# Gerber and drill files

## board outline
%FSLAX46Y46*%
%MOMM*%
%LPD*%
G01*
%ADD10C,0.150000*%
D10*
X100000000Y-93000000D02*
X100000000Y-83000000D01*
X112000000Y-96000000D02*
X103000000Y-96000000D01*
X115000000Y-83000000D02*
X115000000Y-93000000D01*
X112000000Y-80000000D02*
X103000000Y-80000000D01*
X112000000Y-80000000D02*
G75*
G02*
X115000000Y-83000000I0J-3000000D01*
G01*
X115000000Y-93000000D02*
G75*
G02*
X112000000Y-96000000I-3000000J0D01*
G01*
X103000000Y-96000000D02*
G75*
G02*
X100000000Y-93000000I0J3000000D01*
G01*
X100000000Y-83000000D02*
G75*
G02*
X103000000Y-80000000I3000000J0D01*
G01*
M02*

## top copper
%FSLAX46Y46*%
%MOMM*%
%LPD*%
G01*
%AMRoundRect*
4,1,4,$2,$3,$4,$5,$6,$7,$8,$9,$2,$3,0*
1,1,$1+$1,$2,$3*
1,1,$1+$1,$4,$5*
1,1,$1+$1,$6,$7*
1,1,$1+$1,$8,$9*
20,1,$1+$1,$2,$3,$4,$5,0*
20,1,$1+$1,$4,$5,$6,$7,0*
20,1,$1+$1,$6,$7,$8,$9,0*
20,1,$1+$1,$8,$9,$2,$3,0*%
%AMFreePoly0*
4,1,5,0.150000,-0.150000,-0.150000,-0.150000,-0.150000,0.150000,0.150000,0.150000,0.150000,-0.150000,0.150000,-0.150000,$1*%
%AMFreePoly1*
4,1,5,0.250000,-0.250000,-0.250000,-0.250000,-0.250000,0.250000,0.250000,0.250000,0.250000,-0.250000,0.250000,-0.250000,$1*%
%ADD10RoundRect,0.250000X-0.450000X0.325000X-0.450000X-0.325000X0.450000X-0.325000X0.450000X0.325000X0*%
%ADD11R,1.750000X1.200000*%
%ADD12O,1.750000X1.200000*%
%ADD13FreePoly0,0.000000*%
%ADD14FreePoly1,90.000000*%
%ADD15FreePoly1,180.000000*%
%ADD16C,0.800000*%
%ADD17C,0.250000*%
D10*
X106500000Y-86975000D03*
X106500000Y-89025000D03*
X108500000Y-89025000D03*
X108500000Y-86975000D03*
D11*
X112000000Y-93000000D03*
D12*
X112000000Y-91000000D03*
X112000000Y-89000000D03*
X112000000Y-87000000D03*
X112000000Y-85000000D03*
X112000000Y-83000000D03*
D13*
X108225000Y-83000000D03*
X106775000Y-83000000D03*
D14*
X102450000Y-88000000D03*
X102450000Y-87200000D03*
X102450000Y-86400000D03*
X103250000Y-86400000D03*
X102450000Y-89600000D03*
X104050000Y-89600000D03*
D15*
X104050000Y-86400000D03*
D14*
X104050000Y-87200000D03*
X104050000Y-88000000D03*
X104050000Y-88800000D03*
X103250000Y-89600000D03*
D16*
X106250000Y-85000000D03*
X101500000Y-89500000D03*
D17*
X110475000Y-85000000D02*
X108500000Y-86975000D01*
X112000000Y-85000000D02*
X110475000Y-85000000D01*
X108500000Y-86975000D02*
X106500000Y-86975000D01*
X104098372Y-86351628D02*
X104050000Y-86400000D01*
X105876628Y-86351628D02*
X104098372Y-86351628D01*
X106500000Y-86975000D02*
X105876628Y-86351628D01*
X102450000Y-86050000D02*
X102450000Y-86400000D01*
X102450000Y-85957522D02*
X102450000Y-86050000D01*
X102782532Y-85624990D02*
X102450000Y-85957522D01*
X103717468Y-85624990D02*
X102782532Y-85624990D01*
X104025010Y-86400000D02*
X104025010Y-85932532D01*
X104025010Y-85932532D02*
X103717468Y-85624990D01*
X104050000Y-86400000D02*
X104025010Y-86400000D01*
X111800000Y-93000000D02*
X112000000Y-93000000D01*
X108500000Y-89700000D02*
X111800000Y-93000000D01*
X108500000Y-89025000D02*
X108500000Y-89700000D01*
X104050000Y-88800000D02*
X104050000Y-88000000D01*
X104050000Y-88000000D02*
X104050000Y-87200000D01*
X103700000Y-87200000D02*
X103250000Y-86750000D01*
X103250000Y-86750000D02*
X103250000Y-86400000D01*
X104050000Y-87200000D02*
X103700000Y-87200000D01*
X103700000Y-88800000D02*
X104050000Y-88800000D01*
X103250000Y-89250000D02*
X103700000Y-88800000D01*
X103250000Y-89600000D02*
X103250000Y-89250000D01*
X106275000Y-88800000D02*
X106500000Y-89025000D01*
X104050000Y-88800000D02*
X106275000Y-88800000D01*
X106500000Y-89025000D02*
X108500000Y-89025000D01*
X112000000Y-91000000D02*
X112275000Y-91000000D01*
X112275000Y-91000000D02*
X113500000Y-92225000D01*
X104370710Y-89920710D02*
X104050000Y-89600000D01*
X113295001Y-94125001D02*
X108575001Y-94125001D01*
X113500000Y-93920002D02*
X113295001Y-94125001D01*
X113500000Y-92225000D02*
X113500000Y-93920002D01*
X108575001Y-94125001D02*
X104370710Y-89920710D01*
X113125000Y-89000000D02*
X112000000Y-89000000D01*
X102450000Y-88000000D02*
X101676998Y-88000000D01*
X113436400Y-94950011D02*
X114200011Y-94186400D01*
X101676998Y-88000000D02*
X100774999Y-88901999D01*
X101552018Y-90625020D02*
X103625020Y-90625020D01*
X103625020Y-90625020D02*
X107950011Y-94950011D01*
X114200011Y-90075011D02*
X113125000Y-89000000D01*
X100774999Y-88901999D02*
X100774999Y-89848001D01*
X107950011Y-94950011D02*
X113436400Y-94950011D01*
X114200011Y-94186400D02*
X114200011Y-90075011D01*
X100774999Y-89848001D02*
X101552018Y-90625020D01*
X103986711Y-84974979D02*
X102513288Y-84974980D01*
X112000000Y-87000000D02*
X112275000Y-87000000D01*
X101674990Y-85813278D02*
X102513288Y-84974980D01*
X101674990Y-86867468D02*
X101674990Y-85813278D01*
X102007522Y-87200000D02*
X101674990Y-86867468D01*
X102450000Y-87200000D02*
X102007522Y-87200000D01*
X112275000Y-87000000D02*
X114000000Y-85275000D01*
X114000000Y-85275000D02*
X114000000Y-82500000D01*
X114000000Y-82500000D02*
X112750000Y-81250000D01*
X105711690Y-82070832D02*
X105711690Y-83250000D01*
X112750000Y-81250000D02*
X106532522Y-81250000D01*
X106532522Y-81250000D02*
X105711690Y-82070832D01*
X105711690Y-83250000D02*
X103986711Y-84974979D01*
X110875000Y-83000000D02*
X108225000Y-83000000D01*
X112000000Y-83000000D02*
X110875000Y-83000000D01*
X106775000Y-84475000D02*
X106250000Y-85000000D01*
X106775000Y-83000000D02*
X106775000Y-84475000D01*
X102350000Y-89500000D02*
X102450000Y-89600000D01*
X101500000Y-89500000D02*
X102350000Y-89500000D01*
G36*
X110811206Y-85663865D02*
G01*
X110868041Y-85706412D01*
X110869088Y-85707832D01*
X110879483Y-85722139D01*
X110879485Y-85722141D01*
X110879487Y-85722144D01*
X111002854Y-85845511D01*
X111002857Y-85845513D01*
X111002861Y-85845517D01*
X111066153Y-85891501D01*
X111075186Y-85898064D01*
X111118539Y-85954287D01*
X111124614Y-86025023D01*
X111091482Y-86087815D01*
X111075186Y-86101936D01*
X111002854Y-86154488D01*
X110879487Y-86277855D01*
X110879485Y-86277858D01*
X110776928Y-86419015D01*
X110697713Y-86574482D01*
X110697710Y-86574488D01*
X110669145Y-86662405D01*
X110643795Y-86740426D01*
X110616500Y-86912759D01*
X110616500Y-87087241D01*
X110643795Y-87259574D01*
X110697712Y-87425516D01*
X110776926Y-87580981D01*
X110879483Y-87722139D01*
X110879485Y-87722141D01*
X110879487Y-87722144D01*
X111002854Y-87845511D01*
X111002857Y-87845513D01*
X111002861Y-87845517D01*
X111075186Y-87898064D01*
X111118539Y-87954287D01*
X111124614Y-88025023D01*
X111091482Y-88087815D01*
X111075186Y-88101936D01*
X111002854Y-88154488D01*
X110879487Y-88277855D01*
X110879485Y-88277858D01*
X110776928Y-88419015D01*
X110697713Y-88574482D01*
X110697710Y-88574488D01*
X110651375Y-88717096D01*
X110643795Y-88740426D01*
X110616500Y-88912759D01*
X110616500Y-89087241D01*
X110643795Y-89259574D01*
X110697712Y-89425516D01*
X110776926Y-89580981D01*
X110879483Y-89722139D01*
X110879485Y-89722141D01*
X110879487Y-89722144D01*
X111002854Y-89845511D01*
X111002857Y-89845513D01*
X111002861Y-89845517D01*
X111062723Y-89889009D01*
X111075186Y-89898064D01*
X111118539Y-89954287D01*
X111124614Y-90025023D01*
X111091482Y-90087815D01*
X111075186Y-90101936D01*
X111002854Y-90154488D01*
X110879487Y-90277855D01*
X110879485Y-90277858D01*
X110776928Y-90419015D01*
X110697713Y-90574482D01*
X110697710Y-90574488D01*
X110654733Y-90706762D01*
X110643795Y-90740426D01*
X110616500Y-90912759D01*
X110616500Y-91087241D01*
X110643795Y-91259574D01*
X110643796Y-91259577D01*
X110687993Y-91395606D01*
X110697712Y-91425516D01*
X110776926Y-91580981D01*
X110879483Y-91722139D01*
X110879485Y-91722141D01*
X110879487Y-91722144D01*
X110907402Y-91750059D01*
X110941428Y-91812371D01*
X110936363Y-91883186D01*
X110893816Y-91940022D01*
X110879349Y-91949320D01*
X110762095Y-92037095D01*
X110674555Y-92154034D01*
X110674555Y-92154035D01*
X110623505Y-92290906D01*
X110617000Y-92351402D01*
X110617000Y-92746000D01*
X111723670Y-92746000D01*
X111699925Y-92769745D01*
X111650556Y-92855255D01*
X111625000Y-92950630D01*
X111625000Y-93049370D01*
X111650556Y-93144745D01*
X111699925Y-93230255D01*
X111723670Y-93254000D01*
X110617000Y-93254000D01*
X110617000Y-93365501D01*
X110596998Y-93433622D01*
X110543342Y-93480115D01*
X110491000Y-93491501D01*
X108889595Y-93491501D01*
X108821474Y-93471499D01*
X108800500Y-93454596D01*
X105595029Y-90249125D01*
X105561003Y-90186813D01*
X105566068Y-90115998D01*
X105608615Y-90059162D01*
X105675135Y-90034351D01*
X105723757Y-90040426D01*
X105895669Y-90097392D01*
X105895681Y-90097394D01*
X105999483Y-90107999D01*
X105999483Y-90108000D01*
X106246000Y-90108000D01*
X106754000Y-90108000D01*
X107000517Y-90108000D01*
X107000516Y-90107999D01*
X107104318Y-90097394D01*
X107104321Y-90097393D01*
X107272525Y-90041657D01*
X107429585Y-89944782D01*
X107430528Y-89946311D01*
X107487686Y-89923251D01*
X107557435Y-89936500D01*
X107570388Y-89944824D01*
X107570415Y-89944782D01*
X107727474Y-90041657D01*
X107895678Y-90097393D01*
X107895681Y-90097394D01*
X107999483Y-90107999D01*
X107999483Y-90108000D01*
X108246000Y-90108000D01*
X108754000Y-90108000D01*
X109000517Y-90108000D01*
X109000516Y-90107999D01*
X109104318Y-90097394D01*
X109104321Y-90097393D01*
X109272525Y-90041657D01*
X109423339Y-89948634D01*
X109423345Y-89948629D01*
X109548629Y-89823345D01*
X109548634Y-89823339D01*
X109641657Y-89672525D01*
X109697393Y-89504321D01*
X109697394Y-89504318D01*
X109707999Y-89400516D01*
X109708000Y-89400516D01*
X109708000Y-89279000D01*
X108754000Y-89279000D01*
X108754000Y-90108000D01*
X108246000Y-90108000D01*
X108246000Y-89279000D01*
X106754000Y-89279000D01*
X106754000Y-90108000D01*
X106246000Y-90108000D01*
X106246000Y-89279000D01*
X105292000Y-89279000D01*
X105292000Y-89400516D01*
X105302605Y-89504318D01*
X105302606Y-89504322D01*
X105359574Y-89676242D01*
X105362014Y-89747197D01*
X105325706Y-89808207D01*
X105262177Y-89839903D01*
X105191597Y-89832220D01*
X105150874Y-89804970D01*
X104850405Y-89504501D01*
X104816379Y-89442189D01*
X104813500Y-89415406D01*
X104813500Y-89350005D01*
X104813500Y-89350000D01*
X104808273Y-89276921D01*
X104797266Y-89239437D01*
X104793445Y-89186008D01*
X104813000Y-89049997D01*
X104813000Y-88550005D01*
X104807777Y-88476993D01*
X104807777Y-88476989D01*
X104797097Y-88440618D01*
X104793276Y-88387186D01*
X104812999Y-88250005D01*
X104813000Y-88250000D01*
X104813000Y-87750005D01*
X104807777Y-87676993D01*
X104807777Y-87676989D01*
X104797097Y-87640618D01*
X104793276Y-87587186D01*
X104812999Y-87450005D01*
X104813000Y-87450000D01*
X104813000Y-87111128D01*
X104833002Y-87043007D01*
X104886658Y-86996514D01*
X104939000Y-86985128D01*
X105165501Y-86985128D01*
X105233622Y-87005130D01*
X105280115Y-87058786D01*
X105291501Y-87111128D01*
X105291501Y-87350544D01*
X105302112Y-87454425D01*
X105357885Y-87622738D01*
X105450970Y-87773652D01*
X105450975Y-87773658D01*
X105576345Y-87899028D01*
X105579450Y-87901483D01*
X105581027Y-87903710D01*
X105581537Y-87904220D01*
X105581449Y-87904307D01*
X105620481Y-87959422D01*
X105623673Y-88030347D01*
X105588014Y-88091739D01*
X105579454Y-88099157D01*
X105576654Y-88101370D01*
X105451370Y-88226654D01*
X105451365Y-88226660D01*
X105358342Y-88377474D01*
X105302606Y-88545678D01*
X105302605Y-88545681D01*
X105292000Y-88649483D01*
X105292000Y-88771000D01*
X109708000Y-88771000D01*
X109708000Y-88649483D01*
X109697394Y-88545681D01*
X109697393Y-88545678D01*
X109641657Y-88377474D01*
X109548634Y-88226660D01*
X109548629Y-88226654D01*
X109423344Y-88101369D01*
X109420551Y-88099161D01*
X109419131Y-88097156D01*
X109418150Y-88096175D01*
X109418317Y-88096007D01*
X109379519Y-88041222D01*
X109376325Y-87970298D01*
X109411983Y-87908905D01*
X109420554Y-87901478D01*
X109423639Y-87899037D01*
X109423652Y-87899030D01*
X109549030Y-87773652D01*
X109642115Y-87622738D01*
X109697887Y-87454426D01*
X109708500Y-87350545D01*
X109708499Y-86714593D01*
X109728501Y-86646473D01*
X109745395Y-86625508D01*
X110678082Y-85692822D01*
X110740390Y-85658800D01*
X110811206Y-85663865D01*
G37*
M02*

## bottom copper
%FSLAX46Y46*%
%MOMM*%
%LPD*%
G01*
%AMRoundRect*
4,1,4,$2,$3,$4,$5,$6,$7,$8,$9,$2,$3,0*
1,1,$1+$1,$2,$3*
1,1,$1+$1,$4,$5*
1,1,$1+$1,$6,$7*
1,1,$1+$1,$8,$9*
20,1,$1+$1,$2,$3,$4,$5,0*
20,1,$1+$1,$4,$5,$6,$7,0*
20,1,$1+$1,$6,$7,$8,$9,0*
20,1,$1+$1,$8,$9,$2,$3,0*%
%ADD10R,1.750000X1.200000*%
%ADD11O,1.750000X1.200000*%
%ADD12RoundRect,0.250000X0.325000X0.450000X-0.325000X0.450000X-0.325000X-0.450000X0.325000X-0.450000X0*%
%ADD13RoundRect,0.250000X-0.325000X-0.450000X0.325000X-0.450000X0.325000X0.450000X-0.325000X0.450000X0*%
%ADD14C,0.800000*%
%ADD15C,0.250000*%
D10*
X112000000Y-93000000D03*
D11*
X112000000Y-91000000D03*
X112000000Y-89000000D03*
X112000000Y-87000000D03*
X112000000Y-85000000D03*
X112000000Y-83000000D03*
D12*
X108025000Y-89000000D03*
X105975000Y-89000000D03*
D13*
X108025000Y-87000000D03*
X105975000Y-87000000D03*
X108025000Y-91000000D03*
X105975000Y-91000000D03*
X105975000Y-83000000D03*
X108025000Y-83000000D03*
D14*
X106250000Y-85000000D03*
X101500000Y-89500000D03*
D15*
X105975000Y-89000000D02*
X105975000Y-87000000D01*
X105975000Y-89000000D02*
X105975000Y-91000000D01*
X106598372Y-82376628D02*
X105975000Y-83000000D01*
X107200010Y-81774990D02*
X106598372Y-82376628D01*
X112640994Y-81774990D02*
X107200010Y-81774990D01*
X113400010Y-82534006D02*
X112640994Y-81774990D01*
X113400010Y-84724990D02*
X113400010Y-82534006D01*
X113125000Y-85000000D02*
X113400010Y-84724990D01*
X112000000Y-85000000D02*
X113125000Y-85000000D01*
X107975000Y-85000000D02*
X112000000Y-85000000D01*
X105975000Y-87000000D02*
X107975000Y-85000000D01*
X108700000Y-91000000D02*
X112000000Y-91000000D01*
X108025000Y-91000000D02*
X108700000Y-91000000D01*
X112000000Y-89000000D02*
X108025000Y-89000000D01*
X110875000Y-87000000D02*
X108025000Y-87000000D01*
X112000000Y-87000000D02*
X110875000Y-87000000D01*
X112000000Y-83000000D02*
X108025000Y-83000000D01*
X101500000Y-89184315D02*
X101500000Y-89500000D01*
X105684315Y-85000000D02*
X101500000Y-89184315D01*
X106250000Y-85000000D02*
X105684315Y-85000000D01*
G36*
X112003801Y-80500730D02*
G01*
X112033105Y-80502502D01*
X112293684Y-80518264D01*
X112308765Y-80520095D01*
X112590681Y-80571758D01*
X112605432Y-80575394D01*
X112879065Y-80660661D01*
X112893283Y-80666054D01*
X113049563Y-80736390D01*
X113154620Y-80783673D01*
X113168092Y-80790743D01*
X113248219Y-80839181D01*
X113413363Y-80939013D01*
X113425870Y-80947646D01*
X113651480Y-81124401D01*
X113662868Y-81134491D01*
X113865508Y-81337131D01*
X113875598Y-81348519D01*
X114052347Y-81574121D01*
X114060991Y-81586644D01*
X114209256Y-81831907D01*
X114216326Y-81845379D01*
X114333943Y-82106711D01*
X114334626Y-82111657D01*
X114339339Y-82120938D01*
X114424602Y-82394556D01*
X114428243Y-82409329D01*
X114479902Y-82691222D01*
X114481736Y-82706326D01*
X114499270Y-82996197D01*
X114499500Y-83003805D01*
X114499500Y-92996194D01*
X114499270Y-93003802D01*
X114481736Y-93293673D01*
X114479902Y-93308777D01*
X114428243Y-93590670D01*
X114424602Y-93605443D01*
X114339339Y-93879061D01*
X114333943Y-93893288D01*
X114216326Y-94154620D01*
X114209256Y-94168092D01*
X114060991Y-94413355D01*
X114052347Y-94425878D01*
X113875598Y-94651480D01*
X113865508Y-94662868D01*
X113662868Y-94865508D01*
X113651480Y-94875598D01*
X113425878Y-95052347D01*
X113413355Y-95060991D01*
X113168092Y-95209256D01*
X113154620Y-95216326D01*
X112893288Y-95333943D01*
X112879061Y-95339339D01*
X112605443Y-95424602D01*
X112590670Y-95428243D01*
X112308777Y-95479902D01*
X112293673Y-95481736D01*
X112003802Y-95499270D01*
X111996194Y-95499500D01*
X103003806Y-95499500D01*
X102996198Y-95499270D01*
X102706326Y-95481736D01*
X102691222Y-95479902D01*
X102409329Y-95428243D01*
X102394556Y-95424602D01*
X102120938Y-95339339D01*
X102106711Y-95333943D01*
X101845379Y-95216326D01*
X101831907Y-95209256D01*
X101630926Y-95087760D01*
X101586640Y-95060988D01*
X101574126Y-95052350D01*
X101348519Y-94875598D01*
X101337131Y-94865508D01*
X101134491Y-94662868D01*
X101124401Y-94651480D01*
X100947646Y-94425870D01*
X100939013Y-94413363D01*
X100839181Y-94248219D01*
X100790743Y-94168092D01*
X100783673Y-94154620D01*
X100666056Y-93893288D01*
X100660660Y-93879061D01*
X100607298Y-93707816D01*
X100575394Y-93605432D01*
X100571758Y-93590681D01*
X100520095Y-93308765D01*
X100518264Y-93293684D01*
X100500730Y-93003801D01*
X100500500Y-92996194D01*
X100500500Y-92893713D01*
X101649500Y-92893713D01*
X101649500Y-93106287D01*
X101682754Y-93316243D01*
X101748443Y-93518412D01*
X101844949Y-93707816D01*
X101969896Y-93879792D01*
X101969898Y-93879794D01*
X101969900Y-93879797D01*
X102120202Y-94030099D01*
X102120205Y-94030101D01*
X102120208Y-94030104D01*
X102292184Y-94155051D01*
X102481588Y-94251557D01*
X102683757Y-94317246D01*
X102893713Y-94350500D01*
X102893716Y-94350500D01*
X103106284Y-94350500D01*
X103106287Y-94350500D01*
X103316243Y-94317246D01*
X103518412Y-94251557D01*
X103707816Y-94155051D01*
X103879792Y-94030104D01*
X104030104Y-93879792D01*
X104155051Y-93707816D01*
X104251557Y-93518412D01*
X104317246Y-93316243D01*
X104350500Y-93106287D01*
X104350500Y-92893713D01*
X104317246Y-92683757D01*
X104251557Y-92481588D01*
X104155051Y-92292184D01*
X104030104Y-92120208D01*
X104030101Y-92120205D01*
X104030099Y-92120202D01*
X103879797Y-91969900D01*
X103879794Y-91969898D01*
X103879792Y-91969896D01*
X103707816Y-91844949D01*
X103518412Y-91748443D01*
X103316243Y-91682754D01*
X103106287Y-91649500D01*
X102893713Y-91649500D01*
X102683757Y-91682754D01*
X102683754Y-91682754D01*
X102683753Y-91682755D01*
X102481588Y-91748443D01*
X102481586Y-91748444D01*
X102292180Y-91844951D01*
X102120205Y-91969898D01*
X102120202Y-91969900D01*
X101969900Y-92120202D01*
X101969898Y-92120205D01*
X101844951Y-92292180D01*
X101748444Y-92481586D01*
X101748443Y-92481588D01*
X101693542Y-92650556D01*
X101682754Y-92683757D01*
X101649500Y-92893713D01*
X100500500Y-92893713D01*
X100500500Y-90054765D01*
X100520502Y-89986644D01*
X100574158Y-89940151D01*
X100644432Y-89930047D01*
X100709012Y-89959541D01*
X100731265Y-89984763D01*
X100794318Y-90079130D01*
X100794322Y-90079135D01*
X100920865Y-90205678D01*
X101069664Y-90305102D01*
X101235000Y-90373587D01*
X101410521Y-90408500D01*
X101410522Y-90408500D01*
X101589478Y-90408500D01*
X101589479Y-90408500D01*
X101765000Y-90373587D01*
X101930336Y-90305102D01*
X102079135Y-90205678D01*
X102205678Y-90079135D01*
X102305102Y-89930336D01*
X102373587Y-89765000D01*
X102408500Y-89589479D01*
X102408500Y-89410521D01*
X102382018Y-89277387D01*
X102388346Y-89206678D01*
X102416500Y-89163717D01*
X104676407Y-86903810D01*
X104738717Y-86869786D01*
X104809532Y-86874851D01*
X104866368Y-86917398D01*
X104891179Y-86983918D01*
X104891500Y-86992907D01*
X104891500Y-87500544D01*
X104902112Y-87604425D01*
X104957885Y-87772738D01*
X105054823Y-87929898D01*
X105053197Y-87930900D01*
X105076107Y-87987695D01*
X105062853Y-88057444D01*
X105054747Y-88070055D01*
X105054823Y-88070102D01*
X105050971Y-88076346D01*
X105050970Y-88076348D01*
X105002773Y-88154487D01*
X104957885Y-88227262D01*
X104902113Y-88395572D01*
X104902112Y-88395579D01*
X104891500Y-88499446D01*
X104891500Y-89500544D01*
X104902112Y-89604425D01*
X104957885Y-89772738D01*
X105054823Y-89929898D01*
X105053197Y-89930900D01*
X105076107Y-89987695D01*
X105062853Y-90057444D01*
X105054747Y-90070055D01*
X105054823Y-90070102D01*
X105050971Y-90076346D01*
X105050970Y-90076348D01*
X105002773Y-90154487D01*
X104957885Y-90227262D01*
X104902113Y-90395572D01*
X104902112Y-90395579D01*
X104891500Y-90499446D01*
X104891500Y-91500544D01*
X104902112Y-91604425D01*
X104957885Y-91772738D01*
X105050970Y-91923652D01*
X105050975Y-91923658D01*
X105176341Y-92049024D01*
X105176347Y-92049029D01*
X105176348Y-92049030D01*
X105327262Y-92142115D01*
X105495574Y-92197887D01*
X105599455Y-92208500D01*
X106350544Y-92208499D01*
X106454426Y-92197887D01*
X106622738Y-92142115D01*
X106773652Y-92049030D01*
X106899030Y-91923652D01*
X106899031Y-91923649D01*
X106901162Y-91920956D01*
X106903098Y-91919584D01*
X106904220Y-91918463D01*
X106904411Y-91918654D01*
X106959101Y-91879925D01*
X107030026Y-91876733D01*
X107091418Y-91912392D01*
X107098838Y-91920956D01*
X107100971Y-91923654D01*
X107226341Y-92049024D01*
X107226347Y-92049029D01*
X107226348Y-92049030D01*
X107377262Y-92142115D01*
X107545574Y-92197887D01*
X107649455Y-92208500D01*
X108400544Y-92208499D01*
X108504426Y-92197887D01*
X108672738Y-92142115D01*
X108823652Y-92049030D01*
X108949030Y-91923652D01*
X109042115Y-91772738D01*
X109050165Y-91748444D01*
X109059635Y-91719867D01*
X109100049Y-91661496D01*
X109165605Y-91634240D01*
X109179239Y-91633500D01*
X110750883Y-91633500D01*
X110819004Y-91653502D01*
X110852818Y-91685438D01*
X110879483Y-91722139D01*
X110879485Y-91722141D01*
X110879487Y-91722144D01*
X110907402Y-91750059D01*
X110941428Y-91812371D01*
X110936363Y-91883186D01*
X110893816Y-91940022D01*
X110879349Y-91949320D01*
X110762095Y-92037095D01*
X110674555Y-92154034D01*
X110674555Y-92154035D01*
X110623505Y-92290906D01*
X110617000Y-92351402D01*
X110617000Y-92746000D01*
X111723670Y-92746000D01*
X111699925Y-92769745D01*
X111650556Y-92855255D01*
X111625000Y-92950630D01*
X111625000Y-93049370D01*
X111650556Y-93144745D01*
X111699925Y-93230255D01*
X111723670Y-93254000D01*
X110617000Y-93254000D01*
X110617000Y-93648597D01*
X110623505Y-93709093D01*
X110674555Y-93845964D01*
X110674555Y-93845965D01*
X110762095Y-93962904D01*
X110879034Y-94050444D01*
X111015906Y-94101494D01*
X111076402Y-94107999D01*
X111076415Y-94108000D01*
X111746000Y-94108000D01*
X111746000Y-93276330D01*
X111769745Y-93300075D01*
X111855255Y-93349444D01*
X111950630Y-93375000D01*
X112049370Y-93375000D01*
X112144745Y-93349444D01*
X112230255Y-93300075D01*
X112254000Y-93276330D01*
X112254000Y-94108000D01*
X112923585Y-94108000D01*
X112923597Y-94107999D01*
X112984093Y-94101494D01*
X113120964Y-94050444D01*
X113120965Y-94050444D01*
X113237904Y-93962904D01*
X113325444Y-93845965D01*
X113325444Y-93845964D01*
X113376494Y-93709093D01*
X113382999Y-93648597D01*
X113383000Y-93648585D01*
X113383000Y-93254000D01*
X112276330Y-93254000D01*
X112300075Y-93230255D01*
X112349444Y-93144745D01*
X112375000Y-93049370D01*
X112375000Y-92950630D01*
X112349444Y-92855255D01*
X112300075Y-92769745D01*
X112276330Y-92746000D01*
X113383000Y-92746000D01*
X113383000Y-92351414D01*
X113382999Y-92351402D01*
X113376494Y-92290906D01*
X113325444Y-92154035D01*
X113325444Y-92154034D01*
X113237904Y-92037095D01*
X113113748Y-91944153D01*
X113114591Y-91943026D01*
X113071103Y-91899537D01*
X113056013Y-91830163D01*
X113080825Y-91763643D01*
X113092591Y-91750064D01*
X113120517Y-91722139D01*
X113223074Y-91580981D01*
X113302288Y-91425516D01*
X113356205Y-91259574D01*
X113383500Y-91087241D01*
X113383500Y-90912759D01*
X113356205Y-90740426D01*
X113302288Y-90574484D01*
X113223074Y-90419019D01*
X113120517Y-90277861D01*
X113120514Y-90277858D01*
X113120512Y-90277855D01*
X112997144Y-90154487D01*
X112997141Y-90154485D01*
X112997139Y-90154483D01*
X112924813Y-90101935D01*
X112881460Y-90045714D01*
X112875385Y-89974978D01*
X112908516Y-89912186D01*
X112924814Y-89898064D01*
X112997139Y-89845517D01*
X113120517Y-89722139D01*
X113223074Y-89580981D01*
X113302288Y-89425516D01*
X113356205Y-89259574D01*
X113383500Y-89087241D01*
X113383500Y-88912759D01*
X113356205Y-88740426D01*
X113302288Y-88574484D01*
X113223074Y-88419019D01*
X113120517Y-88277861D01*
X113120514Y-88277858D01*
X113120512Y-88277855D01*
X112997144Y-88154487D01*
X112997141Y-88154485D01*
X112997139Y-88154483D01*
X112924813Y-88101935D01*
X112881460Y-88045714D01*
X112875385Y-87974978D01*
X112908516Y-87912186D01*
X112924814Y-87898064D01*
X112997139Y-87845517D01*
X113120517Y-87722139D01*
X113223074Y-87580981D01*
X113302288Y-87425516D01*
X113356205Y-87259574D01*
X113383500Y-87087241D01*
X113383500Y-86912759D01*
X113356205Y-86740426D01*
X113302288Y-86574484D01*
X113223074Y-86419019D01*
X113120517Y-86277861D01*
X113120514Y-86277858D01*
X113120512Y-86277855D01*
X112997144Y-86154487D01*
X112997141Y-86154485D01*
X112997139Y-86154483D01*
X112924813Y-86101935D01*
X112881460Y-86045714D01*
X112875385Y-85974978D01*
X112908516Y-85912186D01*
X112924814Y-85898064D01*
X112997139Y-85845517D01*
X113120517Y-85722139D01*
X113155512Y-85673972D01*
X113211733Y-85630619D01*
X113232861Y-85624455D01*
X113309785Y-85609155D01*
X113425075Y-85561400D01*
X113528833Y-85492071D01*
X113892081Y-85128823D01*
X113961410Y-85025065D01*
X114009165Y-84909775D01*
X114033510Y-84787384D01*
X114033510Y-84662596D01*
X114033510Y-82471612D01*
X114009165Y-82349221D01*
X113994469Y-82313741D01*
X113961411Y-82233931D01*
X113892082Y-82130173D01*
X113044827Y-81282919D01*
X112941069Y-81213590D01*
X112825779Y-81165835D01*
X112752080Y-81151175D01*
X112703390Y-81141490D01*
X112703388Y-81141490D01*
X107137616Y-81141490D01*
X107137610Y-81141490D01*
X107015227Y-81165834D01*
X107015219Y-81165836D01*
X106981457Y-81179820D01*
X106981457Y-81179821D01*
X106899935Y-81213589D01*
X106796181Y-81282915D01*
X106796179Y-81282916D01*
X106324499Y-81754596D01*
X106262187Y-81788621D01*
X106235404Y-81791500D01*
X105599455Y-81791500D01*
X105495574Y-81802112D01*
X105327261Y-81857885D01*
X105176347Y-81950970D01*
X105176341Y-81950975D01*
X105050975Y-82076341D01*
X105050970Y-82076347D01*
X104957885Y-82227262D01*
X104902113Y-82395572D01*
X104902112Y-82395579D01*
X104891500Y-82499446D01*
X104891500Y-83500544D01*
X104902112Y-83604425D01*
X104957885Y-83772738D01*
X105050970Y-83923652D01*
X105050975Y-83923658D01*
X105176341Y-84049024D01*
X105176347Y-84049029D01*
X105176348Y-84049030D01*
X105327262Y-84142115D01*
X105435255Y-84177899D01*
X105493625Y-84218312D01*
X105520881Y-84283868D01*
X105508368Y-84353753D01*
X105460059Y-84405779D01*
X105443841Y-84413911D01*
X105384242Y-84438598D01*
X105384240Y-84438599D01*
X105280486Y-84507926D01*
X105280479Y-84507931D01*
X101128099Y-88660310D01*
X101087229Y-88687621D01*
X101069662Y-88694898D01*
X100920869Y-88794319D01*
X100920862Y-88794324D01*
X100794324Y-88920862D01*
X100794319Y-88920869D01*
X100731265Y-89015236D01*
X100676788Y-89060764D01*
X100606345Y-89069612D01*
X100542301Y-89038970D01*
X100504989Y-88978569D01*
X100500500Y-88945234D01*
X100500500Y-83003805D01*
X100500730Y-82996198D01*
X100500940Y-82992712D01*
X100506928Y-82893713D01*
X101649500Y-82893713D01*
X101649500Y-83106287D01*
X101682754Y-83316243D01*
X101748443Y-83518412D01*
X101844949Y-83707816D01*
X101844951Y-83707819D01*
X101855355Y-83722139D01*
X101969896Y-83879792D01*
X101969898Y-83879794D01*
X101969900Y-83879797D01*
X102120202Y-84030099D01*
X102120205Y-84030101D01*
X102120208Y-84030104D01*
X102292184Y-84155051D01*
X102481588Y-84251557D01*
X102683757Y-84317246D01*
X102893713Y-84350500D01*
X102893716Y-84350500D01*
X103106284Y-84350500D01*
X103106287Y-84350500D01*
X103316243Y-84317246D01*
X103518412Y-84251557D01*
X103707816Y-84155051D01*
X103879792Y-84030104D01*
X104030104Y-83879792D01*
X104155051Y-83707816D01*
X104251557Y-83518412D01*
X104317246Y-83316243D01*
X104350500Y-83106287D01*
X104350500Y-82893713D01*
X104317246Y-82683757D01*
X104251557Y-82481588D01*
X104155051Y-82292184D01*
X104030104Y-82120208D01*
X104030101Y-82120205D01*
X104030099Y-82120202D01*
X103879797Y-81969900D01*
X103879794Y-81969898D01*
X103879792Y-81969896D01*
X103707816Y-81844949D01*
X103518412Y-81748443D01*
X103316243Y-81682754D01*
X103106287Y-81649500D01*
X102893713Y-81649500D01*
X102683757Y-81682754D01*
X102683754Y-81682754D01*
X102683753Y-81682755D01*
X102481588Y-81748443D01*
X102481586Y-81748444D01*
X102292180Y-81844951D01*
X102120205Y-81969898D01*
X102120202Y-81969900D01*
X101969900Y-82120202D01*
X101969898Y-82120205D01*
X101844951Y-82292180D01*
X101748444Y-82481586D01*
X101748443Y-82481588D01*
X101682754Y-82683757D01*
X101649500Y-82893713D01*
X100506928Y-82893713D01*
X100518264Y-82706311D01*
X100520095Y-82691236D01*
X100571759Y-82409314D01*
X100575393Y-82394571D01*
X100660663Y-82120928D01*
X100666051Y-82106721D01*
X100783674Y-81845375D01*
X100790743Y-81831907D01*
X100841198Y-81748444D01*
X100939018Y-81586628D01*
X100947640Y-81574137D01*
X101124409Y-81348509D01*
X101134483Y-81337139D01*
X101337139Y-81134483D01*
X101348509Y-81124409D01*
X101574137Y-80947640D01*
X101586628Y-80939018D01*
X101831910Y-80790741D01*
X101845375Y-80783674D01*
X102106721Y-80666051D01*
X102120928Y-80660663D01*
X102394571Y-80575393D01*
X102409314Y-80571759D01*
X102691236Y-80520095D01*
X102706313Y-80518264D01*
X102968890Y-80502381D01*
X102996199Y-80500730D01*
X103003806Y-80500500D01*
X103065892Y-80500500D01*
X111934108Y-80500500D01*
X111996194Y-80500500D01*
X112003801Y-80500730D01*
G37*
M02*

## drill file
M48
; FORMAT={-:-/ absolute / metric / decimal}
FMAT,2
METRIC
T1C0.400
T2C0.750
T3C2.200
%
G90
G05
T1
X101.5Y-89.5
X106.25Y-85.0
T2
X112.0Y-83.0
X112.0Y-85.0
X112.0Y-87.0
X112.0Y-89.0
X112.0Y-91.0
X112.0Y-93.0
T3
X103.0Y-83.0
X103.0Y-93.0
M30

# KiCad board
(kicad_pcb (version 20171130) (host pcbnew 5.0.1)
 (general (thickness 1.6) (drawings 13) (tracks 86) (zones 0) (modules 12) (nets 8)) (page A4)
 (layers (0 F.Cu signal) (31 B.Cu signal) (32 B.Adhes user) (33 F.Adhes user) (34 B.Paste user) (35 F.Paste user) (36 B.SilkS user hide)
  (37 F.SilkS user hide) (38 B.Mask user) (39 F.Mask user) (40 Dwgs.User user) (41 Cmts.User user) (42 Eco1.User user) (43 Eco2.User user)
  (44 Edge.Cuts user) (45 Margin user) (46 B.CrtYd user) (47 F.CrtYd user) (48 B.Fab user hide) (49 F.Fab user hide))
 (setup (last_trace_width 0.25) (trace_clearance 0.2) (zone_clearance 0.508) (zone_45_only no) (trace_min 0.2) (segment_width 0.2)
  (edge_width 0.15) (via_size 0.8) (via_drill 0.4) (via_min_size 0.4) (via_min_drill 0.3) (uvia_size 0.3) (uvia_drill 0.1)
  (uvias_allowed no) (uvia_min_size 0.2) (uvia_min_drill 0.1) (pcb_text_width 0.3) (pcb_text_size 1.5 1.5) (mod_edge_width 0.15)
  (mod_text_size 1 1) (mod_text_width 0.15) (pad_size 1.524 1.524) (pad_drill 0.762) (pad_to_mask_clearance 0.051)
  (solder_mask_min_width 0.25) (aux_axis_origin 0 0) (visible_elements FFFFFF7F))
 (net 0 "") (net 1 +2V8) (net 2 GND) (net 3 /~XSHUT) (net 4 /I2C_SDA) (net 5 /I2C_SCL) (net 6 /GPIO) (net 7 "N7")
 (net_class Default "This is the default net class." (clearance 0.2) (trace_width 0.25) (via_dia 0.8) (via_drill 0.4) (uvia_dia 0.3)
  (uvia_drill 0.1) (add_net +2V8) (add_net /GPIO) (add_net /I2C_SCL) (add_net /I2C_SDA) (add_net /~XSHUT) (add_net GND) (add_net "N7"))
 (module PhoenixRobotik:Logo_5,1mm (layer F.Cu) (at 108 93.75 90)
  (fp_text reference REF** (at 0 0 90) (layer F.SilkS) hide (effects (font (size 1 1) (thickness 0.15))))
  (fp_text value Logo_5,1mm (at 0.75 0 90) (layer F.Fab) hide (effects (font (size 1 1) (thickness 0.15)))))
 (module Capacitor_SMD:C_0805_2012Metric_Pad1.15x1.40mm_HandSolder (layer F.Cu) (at 106.5 88 270)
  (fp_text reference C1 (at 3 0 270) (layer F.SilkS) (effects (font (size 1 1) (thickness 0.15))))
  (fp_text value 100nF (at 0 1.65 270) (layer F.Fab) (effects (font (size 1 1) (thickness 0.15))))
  (pad 1 smd roundrect (at -1.025 0 270) (size 1.15 1.4) (layers F.Cu F.Paste F.Mask) (roundrect_rratio 0.217391) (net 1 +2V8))
  (pad 2 smd roundrect (at 1.025 0 270) (size 1.15 1.4) (layers F.Cu F.Paste F.Mask) (roundrect_rratio 0.217391) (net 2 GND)))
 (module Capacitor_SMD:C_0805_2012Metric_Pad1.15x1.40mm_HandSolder (layer F.Cu) (at 108.5 88 270)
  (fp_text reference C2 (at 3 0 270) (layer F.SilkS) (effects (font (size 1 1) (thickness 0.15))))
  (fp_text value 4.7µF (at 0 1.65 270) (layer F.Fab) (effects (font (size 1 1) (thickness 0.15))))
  (pad 2 smd roundrect (at 1.025 0 270) (size 1.15 1.4) (layers F.Cu F.Paste F.Mask) (roundrect_rratio 0.217391) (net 2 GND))
  (pad 1 smd roundrect (at -1.025 0 270) (size 1.15 1.4) (layers F.Cu F.Paste F.Mask) (roundrect_rratio 0.217391) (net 1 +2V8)))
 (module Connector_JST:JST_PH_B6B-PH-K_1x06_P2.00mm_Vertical (layer B.Cu) (at 112 93 90)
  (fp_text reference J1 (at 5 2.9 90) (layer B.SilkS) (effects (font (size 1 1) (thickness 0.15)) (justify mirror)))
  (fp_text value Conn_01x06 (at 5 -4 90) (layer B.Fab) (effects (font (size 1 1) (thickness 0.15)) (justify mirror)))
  (pad 1 thru_hole rect (at 0 0 90) (size 1.2 1.75) (drill 0.75) (layers *.Cu *.Mask) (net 2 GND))
  (pad 2 thru_hole oval (at 2 0 90) (size 1.2 1.75) (drill 0.75) (layers *.Cu *.Mask) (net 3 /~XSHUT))
  (pad 3 thru_hole oval (at 4 0 90) (size 1.2 1.75) (drill 0.75) (layers *.Cu *.Mask) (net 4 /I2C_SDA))
  (pad 4 thru_hole oval (at 6 0 90) (size 1.2 1.75) (drill 0.75) (layers *.Cu *.Mask) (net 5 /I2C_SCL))
  (pad 5 thru_hole oval (at 8 0 90) (size 1.2 1.75) (drill 0.75) (layers *.Cu *.Mask) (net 1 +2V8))
  (pad 6 thru_hole oval (at 10 0 90) (size 1.2 1.75) (drill 0.75) (layers *.Cu *.Mask) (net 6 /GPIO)))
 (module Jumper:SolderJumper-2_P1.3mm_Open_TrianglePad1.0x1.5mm (layer F.Cu) (at 107.5 83)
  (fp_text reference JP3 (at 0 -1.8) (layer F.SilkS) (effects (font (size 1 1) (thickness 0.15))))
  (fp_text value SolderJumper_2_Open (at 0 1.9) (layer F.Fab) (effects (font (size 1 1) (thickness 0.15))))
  (pad 2 smd custom (at 0.725 0) (size 0.3 0.3) (layers F.Cu F.Mask) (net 6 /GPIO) (zone_connect 0)
   (options (clearance outline) (anchor rect)) (primitives))
  (pad 1 smd custom (at -0.725 0) (size 0.3 0.3) (layers F.Cu F.Mask) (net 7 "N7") (zone_connect 0)
   (options (clearance outline) (anchor rect)) (primitives)))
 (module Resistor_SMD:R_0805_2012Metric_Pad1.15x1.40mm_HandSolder (layer B.Cu) (at 107 89 180)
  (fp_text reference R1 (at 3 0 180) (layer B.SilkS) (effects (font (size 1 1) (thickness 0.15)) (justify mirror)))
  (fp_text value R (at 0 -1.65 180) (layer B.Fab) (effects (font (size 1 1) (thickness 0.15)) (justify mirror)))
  (pad 1 smd roundrect (at -1.025 0 180) (size 1.15 1.4) (layers B.Cu B.Paste B.Mask) (roundrect_rratio 0.217391) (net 4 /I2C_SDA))
  (pad 2 smd roundrect (at 1.025 0 180) (size 1.15 1.4) (layers B.Cu B.Paste B.Mask) (roundrect_rratio 0.217391) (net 1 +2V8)))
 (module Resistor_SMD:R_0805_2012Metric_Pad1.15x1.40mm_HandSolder (layer B.Cu) (at 107 87)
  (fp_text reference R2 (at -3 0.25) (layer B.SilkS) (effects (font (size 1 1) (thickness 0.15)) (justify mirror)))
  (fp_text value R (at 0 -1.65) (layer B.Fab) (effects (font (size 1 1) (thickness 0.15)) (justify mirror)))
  (pad 2 smd roundrect (at 1.025 0) (size 1.15 1.4) (layers B.Cu B.Paste B.Mask) (roundrect_rratio 0.217391) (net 5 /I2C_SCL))
  (pad 1 smd roundrect (at -1.025 0) (size 1.15 1.4) (layers B.Cu B.Paste B.Mask) (roundrect_rratio 0.217391) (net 1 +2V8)))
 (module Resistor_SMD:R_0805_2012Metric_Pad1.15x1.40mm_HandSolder (layer B.Cu) (at 107 91)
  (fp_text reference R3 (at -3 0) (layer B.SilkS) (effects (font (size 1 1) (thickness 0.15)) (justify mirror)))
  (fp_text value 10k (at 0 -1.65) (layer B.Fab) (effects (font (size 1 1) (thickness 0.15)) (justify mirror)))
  (pad 2 smd roundrect (at 1.025 0) (size 1.15 1.4) (layers B.Cu B.Paste B.Mask) (roundrect_rratio 0.217391) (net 3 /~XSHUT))
  (pad 1 smd roundrect (at -1.025 0) (size 1.15 1.4) (layers B.Cu B.Paste B.Mask) (roundrect_rratio 0.217391) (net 1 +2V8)))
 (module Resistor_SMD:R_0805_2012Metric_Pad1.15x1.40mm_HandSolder (layer B.Cu) (at 107 83)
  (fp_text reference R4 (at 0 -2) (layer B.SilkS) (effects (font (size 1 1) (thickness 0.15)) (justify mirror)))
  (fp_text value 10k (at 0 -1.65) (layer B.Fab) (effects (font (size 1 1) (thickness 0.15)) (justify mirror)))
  (pad 1 smd roundrect (at -1.025 0) (size 1.15 1.4) (layers B.Cu B.Paste B.Mask) (roundrect_rratio 0.217391) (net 1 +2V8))
  (pad 2 smd roundrect (at 1.025 0) (size 1.15 1.4) (layers B.Cu B.Paste B.Mask) (roundrect_rratio 0.217391) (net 6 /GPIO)))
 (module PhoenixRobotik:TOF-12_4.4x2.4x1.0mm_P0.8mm (layer F.Cu) (at 103.25 88 90)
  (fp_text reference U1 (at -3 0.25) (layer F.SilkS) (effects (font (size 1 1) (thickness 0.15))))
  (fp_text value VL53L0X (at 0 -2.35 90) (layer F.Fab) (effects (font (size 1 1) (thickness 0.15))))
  (pad 2 smd custom (at 0 -0.8 90) (size 0.5 0.5) (layers F.Cu F.Paste F.Mask) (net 4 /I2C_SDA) (zone_connect 0)
   (options (clearance outline) (anchor rect)) (primitives))
  (pad 3 smd custom (at 0.8 -0.8 90) (size 0.5 0.5) (layers F.Cu F.Paste F.Mask) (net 5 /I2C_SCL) (zone_connect 0)
   (options (clearance outline) (anchor rect)) (primitives))
  (pad 1 smd custom (at 1.6 -0.8 90) (size 0.5 0.5) (layers F.Cu F.Paste F.Mask) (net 1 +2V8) (zone_connect 0)
   (options (clearance outline) (anchor rect)) (primitives))
  (pad 4 smd custom (at 1.6 0 90) (size 0.5 0.5) (layers F.Cu F.Paste F.Mask) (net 2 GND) (zone_connect 0)
   (options (clearance outline) (anchor rect)) (primitives))
  (pad 6 smd custom (at -1.6 -0.8 90) (size 0.5 0.5) (layers F.Cu F.Paste F.Mask) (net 7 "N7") (zone_connect 0)
   (options (clearance outline) (anchor rect)) (primitives))
  (pad 5 smd custom (at -1.6 0.8 90) (size 0.5 0.5) (layers F.Cu F.Paste F.Mask) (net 3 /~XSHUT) (zone_connect 0)
   (options (clearance outline) (anchor rect)) (primitives))
  (pad 1 smd custom (at 1.6 0.8 180) (size 0.5 0.5) (layers F.Cu F.Paste F.Mask) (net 1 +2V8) (zone_connect 0)
   (options (clearance outline) (anchor rect)) (primitives))
  (pad 4 smd custom (at 0.8 0.8 90) (size 0.5 0.5) (layers F.Cu F.Paste F.Mask) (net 2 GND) (zone_connect 0)
   (options (clearance outline) (anchor rect)) (primitives))
  (pad 4 smd custom (at 0 0.8 90) (size 0.5 0.5) (layers F.Cu F.Paste F.Mask) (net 2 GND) (zone_connect 0)
   (options (clearance outline) (anchor rect)) (primitives))
  (pad 4 smd custom (at -0.8 0.8 90) (size 0.5 0.5) (layers F.Cu F.Paste F.Mask) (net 2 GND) (zone_connect 0)
   (options (clearance outline) (anchor rect)) (primitives))
  (pad 4 smd custom (at -1.6 0 90) (size 0.5 0.5) (layers F.Cu F.Paste F.Mask) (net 2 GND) (zone_connect 0)
   (options (clearance outline) (anchor rect)) (primitives)))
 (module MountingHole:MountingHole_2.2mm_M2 (layer F.Cu) (at 103 83)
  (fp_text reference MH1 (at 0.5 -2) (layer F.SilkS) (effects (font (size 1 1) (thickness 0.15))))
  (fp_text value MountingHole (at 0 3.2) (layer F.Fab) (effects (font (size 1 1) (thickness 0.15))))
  (pad 1 np_thru_hole circle (at 0 0) (size 2.2 2.2) (drill 2.2) (layers *.Cu *.Mask)))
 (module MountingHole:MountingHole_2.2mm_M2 (layer F.Cu) (at 103 93)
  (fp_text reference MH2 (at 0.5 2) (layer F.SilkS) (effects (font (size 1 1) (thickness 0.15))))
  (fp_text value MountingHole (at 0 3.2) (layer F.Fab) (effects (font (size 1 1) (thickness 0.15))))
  (pad 1 np_thru_hole circle (at 0 0) (size 2.2 2.2) (drill 2.2) (layers *.Cu *.Mask)))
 (gr_line (start 100 93) (end 100 83) (angle 90) (layer Edge.Cuts) (width 0.15))
 (gr_line (start 112 96) (end 103 96) (angle 90) (layer Edge.Cuts) (width 0.15))
 (gr_line (start 115 83) (end 115 93) (angle 90) (layer Edge.Cuts) (width 0.15))
 (gr_line (start 112 80) (end 103 80) (angle 90) (layer Edge.Cuts) (width 0.15))
 (gr_arc (start 112 83) (end 112 80) (angle 90) (layer Edge.Cuts) (width 0.15))
 (gr_arc (start 112 93) (end 115 93) (angle 90) (layer Edge.Cuts) (width 0.15))
 (gr_arc (start 103 93) (end 103 96) (angle 90) (layer Edge.Cuts) (width 0.15))
 (gr_arc (start 103 83) (end 100 83) (angle 90) (layer Edge.Cuts) (width 0.15))
 (segment (start 110.475 85) (end 108.5 86.975) (width 0.25) (layer F.Cu) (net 1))
 (segment (start 112 85) (end 110.475 85) (width 0.25) (layer F.Cu) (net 1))
 (segment (start 108.5 86.975) (end 106.5 86.975) (width 0.25) (layer F.Cu) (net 1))
 (segment (start 105.975 89) (end 105.975 87) (width 0.25) (layer B.Cu) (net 1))
 (segment (start 105.975 89) (end 105.975 91) (width 0.25) (layer B.Cu) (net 1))
 (segment (start 104.098372 86.351628) (end 104.05 86.4) (width 0.25) (layer F.Cu) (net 1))
 (segment (start 105.876628 86.351628) (end 104.098372 86.351628) (width 0.25) (layer F.Cu) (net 1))
 (segment (start 106.5 86.975) (end 105.876628 86.351628) (width 0.25) (layer F.Cu) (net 1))
 (segment (start 102.45 86.05) (end 102.45 86.4) (width 0.25) (layer F.Cu) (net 1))
 (segment (start 102.45 85.957522) (end 102.45 86.05) (width 0.25) (layer F.Cu) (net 1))
 (segment (start 102.782532 85.62499) (end 102.45 85.957522) (width 0.25) (layer F.Cu) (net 1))
 (segment (start 103.717468 85.62499) (end 102.782532 85.62499) (width 0.25) (layer F.Cu) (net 1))
 (segment (start 104.02501 86.4) (end 104.02501 85.932532) (width 0.25) (layer F.Cu) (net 1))
 (segment (start 104.02501 85.932532) (end 103.717468 85.62499) (width 0.25) (layer F.Cu) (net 1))
 (segment (start 104.05 86.4) (end 104.02501 86.4) (width 0.25) (layer F.Cu) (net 1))
 (segment (start 106.598372 82.376628) (end 105.975 83) (width 0.25) (layer B.Cu) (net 1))
 (segment (start 107.20001 81.77499) (end 106.598372 82.376628) (width 0.25) (layer B.Cu) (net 1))
 (segment (start 112.640994 81.77499) (end 107.20001 81.77499) (width 0.25) (layer B.Cu) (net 1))
 (segment (start 113.40001 82.534006) (end 112.640994 81.77499) (width 0.25) (layer B.Cu) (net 1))
 (segment (start 113.40001 84.72499) (end 113.40001 82.534006) (width 0.25) (layer B.Cu) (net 1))
 (segment (start 113.125 85) (end 113.40001 84.72499) (width 0.25) (layer B.Cu) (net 1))
 (segment (start 112 85) (end 113.125 85) (width 0.25) (layer B.Cu) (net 1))
 (segment (start 107.975 85) (end 112 85) (width 0.25) (layer B.Cu) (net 1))
 (segment (start 105.975 87) (end 107.975 85) (width 0.25) (layer B.Cu) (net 1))
 (segment (start 111.8 93) (end 112 93) (width 0.25) (layer F.Cu) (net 2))
 (segment (start 108.5 89.7) (end 111.8 93) (width 0.25) (layer F.Cu) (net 2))
 (segment (start 108.5 89.025) (end 108.5 89.7) (width 0.25) (layer F.Cu) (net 2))
 (segment (start 104.05 88.8) (end 104.05 88) (width 0.25) (layer F.Cu) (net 2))
 (segment (start 104.05 88) (end 104.05 87.2) (width 0.25) (layer F.Cu) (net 2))
 (segment (start 103.7 87.2) (end 103.25 86.75) (width 0.25) (layer F.Cu) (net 2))
 (segment (start 103.25 86.75) (end 103.25 86.4) (width 0.25) (layer F.Cu) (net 2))
 (segment (start 104.05 87.2) (end 103.7 87.2) (width 0.25) (layer F.Cu) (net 2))
 (segment (start 103.7 88.8) (end 104.05 88.8) (width 0.25) (layer F.Cu) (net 2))
 (segment (start 103.25 89.25) (end 103.7 88.8) (width 0.25) (layer F.Cu) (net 2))
 (segment (start 103.25 89.6) (end 103.25 89.25) (width 0.25) (layer F.Cu) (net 2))
 (segment (start 106.275 88.8) (end 106.5 89.025) (width 0.25) (layer F.Cu) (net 2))
 (segment (start 104.05 88.8) (end 106.275 88.8) (width 0.25) (layer F.Cu) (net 2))
 (segment (start 106.5 89.025) (end 108.5 89.025) (width 0.25) (layer F.Cu) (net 2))
 (segment (start 108.7 91) (end 112 91) (width 0.25) (layer B.Cu) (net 3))
 (segment (start 108.025 91) (end 108.7 91) (width 0.25) (layer B.Cu) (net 3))
 (segment (start 112 91) (end 112.275 91) (width 0.25) (layer F.Cu) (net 3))
 (segment (start 112.275 91) (end 113.5 92.225) (width 0.25) (layer F.Cu) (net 3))
 (segment (start 104.37071 89.92071) (end 104.05 89.6) (width 0.25) (layer F.Cu) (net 3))
 (segment (start 113.295001 94.125001) (end 108.575001 94.125001) (width 0.25) (layer F.Cu) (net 3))
 (segment (start 113.5 93.920002) (end 113.295001 94.125001) (width 0.25) (layer F.Cu) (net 3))
 (segment (start 113.5 92.225) (end 113.5 93.920002) (width 0.25) (layer F.Cu) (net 3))
 (segment (start 108.575001 94.125001) (end 104.37071 89.92071) (width 0.25) (layer F.Cu) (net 3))
 (segment (start 112 89) (end 108.025 89) (width 0.25) (layer B.Cu) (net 4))
 (segment (start 113.125 89) (end 112 89) (width 0.25) (layer F.Cu) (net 4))
 (segment (start 102.45 88) (end 101.676998 88) (width 0.25) (layer F.Cu) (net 4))
 (segment (start 113.4364 94.950011) (end 114.200011 94.1864) (width 0.25) (layer F.Cu) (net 4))
 (segment (start 101.676998 88) (end 100.774999 88.901999) (width 0.25) (layer F.Cu) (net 4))
 (segment (start 101.552018 90.62502) (end 103.62502 90.62502) (width 0.25) (layer F.Cu) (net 4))
 (segment (start 103.62502 90.62502) (end 107.950011 94.950011) (width 0.25) (layer F.Cu) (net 4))
 (segment (start 114.200011 90.075011) (end 113.125 89) (width 0.25) (layer F.Cu) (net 4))
 (segment (start 100.774999 88.901999) (end 100.774999 89.848001) (width 0.25) (layer F.Cu) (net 4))
 (segment (start 107.950011 94.950011) (end 113.4364 94.950011) (width 0.25) (layer F.Cu) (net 4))
 (segment (start 114.200011 94.1864) (end 114.200011 90.075011) (width 0.25) (layer F.Cu) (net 4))
 (segment (start 100.774999 89.848001) (end 101.552018 90.62502) (width 0.25) (layer F.Cu) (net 4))
 (segment (start 110.875 87) (end 108.025 87) (width 0.25) (layer B.Cu) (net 5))
 (segment (start 112 87) (end 110.875 87) (width 0.25) (layer B.Cu) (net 5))
 (segment (start 103.986711 84.974979) (end 102.513288 84.97498) (width 0.25) (layer F.Cu) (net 5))
 (segment (start 112 87) (end 112.275 87) (width 0.25) (layer F.Cu) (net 5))
 (segment (start 101.67499 85.813278) (end 102.513288 84.97498) (width 0.25) (layer F.Cu) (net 5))
 (segment (start 101.67499 86.867468) (end 101.67499 85.813278) (width 0.25) (layer F.Cu) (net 5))
 (segment (start 102.007522 87.2) (end 101.67499 86.867468) (width 0.25) (layer F.Cu) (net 5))
 (segment (start 102.45 87.2) (end 102.007522 87.2) (width 0.25) (layer F.Cu) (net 5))
 (segment (start 112.275 87) (end 114 85.275) (width 0.25) (layer F.Cu) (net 5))
 (segment (start 114 85.275) (end 114 82.5) (width 0.25) (layer F.Cu) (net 5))
 (segment (start 114 82.5) (end 112.75 81.25) (width 0.25) (layer F.Cu) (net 5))
 (segment (start 105.71169 82.070832) (end 105.71169 83.25) (width 0.25) (layer F.Cu) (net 5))
 (segment (start 112.75 81.25) (end 106.532522 81.25) (width 0.25) (layer F.Cu) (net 5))
 (segment (start 106.532522 81.25) (end 105.71169 82.070832) (width 0.25) (layer F.Cu) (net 5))
 (segment (start 105.71169 83.25) (end 103.986711 84.974979) (width 0.25) (layer F.Cu) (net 5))
 (segment (start 110.875 83) (end 108.225 83) (width 0.25) (layer F.Cu) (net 6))
 (segment (start 112 83) (end 110.875 83) (width 0.25) (layer F.Cu) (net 6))
 (segment (start 112 83) (end 108.025 83) (width 0.25) (layer B.Cu) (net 6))
 (via (at 106.25 85) (size 0.8) (drill 0.4) (layers F.Cu B.Cu) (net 7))
 (via (at 101.5 89.5) (size 0.8) (drill 0.4) (layers F.Cu B.Cu) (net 7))
 (segment (start 106.775 84.475) (end 106.25 85) (width 0.25) (layer F.Cu) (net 7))
 (segment (start 106.775 83) (end 106.775 84.475) (width 0.25) (layer F.Cu) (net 7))
 (segment (start 101.5 89.184315) (end 101.5 89.5) (width 0.25) (layer B.Cu) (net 7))
 (segment (start 105.684315 85) (end 101.5 89.184315) (width 0.25) (layer B.Cu) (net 7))
 (segment (start 106.25 85) (end 105.684315 85) (width 0.25) (layer B.Cu) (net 7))
 (segment (start 102.35 89.5) (end 102.45 89.6) (width 0.25) (layer F.Cu) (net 7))
 (segment (start 101.5 89.5) (end 102.35 89.5) (width 0.25) (layer F.Cu) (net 7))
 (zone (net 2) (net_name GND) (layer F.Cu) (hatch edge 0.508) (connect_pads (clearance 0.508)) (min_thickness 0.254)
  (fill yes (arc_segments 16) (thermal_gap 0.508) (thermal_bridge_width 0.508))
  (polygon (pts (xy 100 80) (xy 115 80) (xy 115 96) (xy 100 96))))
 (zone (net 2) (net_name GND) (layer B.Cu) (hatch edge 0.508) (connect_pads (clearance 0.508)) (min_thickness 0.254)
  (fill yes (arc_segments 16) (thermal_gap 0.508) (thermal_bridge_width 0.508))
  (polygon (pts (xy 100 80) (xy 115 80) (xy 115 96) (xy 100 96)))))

